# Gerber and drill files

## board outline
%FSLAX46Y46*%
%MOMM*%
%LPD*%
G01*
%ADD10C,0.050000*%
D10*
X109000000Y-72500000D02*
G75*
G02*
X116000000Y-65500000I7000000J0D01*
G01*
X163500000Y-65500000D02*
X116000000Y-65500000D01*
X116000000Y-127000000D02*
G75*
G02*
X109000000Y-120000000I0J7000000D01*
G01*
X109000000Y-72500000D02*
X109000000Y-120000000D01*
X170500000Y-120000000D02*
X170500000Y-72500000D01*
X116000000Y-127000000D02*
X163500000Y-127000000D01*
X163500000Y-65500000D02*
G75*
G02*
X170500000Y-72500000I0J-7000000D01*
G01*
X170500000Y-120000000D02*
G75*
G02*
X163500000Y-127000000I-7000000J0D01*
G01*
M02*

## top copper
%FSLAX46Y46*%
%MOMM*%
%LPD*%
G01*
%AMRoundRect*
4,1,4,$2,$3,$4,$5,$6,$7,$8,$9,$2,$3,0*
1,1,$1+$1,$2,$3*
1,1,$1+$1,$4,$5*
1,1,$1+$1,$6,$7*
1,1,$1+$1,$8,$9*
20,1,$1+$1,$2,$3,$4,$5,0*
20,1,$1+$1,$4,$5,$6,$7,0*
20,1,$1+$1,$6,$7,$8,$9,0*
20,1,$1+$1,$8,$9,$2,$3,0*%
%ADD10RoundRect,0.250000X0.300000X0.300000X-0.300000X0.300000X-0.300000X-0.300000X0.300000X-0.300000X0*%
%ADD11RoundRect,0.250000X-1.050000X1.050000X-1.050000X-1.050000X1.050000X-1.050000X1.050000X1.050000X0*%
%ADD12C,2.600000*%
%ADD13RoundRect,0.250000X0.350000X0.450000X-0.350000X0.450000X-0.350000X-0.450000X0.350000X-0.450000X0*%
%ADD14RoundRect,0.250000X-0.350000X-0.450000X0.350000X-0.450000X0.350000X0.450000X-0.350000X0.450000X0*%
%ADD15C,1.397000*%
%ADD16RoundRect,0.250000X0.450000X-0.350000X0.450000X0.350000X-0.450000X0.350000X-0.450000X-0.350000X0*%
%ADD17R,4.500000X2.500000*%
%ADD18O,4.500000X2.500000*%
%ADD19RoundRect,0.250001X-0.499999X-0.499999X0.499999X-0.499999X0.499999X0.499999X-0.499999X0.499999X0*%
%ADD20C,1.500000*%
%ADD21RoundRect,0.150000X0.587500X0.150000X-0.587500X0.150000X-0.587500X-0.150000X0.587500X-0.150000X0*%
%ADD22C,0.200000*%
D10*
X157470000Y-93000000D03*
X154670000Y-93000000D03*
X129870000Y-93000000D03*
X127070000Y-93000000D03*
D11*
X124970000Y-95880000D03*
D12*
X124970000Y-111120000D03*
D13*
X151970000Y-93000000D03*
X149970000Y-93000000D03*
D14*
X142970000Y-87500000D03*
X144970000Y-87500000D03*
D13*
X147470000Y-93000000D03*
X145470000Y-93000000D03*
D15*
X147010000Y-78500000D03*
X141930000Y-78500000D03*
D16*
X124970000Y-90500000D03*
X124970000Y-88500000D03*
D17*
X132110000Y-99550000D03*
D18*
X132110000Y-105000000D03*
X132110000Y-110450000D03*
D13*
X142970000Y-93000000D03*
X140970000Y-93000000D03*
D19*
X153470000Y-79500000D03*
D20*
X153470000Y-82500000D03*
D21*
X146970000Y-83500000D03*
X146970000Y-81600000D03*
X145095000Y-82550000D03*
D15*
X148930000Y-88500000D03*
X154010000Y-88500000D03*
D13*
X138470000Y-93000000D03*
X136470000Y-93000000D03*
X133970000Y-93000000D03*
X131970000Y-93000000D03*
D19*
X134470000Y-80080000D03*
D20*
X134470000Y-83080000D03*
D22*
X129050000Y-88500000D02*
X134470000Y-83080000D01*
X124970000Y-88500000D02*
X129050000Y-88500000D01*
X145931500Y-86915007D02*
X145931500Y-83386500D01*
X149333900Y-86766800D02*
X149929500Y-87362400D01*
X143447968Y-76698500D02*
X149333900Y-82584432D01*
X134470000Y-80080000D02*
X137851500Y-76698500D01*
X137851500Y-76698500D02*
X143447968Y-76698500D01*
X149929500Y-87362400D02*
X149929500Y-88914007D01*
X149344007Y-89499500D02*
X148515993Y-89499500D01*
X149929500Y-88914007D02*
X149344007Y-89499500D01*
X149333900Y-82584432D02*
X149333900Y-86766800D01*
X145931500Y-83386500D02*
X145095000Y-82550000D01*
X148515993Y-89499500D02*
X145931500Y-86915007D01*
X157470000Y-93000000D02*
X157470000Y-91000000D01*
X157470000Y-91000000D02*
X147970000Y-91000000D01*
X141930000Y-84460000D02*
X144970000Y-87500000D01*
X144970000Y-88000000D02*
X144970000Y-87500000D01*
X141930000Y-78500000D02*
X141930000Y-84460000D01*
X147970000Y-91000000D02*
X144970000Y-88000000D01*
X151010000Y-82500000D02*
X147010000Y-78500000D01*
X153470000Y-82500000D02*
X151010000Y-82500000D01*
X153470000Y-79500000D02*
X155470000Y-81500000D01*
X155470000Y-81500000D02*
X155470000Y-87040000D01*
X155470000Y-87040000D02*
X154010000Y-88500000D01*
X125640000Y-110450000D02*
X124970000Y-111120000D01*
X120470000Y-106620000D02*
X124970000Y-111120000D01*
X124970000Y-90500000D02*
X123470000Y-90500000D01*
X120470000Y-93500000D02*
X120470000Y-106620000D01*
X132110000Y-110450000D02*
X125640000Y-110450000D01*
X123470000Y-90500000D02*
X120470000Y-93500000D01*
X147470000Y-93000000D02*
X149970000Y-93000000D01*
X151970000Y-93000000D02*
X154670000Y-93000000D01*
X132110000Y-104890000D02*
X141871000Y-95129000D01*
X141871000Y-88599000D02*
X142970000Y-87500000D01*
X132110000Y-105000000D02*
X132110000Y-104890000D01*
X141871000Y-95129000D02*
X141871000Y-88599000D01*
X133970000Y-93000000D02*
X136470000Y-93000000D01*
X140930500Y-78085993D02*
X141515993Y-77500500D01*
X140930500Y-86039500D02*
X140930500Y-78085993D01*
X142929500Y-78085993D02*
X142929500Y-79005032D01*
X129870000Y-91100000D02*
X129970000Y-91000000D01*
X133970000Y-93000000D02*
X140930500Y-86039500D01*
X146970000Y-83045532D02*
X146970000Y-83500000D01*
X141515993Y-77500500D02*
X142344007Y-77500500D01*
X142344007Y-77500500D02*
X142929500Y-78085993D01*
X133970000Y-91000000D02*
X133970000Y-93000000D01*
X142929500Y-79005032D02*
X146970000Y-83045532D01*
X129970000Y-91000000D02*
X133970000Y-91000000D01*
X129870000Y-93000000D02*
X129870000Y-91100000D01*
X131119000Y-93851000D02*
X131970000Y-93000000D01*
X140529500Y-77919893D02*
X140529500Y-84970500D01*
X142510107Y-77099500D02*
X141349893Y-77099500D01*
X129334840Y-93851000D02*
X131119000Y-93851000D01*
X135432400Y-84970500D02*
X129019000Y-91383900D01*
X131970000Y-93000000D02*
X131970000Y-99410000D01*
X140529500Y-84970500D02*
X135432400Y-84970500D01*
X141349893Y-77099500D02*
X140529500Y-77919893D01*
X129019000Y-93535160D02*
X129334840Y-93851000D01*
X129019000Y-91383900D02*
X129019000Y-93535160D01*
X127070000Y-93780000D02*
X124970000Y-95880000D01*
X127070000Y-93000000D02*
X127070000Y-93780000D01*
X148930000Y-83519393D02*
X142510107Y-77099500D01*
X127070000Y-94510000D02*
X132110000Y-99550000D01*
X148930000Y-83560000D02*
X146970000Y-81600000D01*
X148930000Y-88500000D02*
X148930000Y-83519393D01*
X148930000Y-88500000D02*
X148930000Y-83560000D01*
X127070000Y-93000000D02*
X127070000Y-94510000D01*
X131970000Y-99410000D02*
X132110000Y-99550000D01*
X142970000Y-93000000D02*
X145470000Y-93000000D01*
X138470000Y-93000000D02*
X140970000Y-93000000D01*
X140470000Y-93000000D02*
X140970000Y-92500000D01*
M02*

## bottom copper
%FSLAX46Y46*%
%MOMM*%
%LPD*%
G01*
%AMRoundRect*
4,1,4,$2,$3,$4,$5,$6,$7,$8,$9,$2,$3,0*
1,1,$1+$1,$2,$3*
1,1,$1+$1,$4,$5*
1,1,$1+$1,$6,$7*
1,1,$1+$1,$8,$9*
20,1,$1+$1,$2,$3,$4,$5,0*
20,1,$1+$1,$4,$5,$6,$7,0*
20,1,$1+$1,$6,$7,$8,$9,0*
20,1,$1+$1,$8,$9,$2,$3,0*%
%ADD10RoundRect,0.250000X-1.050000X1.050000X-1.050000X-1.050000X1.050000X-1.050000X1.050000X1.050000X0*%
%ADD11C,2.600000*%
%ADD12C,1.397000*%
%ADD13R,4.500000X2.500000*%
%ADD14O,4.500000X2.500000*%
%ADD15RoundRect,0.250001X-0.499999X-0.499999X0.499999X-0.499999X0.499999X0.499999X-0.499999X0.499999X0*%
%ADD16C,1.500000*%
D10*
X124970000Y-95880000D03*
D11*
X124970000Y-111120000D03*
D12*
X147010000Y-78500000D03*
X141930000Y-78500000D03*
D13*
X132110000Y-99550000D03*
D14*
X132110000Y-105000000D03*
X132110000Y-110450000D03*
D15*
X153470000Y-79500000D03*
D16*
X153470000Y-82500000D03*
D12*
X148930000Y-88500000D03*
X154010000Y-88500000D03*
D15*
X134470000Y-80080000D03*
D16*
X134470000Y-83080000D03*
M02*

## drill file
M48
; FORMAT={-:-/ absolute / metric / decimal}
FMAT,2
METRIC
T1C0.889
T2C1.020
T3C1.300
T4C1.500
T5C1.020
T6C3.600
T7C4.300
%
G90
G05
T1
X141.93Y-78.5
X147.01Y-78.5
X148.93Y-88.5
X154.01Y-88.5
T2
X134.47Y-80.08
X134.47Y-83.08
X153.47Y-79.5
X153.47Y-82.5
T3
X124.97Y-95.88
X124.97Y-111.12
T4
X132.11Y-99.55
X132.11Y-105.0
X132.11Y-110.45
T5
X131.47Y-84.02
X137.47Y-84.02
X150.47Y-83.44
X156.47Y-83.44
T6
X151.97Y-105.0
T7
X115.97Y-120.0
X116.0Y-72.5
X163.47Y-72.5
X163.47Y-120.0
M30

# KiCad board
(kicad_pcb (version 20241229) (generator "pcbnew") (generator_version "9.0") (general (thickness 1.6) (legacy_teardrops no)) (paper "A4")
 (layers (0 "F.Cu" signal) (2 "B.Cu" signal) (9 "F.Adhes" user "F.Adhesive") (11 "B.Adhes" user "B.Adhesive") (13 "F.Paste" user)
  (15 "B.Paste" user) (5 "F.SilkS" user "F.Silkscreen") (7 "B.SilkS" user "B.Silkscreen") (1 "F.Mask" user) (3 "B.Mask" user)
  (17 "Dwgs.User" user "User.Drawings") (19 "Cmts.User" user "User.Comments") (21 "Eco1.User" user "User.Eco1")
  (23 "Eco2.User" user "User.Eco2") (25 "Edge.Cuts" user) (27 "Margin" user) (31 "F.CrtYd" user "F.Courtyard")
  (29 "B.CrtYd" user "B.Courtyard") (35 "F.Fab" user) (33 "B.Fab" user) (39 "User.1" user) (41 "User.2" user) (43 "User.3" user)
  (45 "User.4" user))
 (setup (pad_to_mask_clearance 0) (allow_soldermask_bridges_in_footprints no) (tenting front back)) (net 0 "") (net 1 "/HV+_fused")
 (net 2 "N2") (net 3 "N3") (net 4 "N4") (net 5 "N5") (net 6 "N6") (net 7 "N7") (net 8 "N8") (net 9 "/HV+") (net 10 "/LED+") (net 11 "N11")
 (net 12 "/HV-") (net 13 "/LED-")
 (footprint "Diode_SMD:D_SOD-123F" (layer "F.Cu") (at 156.07 93 180)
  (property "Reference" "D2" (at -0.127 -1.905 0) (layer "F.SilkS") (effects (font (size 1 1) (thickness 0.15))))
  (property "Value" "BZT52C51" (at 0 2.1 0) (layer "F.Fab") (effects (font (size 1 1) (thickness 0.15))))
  (pad "1" smd roundrect (at -1.4 0 180) (size 1.1 1.1) (layers "F.Cu" "F.Mask" "F.Paste") (roundrect_rratio 0.2272727273)
   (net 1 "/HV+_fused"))
  (pad "2" smd roundrect (at 1.4 0 180) (size 1.1 1.1) (layers "F.Cu" "F.Mask" "F.Paste") (roundrect_rratio 0.2272727273) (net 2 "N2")))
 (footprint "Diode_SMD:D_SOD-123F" (layer "F.Cu") (at 128.47 93 180)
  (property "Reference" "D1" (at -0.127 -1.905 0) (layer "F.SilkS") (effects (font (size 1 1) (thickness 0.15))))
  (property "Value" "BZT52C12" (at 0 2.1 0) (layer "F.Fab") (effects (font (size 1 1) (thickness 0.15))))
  (pad "1" smd roundrect (at -1.4 0 180) (size 1.1 1.1) (layers "F.Cu" "F.Mask" "F.Paste") (roundrect_rratio 0.2272727273) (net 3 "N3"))
  (pad "2" smd roundrect (at 1.4 0 180) (size 1.1 1.1) (layers "F.Cu" "F.Mask" "F.Paste") (roundrect_rratio 0.2272727273) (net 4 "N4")))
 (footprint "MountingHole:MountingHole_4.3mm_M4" (layer "F.Cu") (at 116 72.5)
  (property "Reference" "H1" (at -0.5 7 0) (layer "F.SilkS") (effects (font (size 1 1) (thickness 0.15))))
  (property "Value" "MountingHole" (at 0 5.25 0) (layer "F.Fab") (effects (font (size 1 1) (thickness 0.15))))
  (pad "" np_thru_hole circle (at 0 0) (size 4.3 4.3) (drill 4.3) (layers "*.Cu" "*.Mask")))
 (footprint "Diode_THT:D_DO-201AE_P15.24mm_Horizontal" (layer "F.Cu") (at 124.97 95.88 -90)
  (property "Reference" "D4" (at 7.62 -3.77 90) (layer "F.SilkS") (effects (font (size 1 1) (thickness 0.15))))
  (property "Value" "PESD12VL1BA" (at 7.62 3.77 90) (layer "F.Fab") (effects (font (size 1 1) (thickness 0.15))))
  (pad "1" thru_hole roundrect (at 0 0 270) (size 2.6 2.6) (drill 1.3) (layers "*.Cu" "*.Mask") (remove_unused_layers no)
   (roundrect_rratio 0.096154) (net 4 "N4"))
  (pad "2" thru_hole circle (at 15.24 0 270) (size 2.6 2.6) (drill 1.3) (layers "*.Cu" "*.Mask") (remove_unused_layers no) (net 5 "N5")))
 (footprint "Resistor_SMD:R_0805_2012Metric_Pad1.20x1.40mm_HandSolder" (layer "F.Cu") (at 150.97 93 180)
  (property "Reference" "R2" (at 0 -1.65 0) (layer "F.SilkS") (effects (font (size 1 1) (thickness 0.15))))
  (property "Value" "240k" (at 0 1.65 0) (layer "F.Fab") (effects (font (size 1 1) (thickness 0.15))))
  (pad "1" smd roundrect (at -1 0 180) (size 1.2 1.4) (layers "F.Cu" "F.Mask" "F.Paste") (roundrect_rratio 0.208333) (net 2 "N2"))
  (pad "2" smd roundrect (at 1 0 180) (size 1.2 1.4) (layers "F.Cu" "F.Mask" "F.Paste") (roundrect_rratio 0.208333) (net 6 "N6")))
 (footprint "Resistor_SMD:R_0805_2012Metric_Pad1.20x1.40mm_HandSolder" (layer "F.Cu") (at 143.97 87.5)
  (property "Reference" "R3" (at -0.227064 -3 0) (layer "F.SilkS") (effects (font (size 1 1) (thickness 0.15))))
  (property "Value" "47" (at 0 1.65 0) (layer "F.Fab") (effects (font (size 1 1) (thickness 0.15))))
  (pad "1" smd roundrect (at -1 0) (size 1.2 1.4) (layers "F.Cu" "F.Mask" "F.Paste") (roundrect_rratio 0.208333) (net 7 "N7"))
  (pad "2" smd roundrect (at 1 0) (size 1.2 1.4) (layers "F.Cu" "F.Mask" "F.Paste") (roundrect_rratio 0.208333) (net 1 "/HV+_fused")))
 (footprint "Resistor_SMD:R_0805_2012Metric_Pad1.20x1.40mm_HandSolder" (layer "F.Cu") (at 146.47 93 180)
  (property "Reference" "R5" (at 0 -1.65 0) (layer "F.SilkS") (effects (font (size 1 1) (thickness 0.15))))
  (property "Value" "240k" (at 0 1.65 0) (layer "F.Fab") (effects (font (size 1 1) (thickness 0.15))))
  (pad "1" smd roundrect (at -1 0 180) (size 1.2 1.4) (layers "F.Cu" "F.Mask" "F.Paste") (roundrect_rratio 0.208333) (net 6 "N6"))
  (pad "2" smd roundrect (at 1 0 180) (size 1.2 1.4) (layers "F.Cu" "F.Mask" "F.Paste") (roundrect_rratio 0.208333) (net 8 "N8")))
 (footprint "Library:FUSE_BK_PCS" (layer "F.Cu") (at 144.47 78.5 180)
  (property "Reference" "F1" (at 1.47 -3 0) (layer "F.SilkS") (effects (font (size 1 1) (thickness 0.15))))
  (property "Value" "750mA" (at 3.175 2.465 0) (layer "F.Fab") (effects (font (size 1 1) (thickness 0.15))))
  (pad "1" thru_hole circle (at -2.54 0 180) (size 1.397 1.397) (drill 0.889) (layers "*.Cu" "*.Mask") (remove_unused_layers no)
   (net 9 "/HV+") (solder_mask_margin 0.102))
  (pad "2" thru_hole circle (at 2.54 0 180) (size 1.397 1.397) (drill 0.889) (layers "*.Cu" "*.Mask") (remove_unused_layers no)
   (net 1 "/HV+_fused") (solder_mask_margin 0.102)))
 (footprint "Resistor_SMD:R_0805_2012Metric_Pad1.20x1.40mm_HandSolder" (layer "F.Cu") (at 124.97 89.5 90)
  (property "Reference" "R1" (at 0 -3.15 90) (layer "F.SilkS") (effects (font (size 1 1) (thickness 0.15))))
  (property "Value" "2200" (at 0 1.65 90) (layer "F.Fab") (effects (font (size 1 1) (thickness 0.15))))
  (pad "1" smd roundrect (at -1 0 90) (size 1.2 1.4) (layers "F.Cu" "F.Mask" "F.Paste") (roundrect_rratio 0.208333) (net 5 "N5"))
  (pad "2" smd roundrect (at 1 0 90) (size 1.2 1.4) (layers "F.Cu" "F.Mask" "F.Paste") (roundrect_rratio 0.208333) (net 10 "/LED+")))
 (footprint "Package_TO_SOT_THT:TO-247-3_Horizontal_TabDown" (layer "F.Cu") (at 132.11 99.55 -90)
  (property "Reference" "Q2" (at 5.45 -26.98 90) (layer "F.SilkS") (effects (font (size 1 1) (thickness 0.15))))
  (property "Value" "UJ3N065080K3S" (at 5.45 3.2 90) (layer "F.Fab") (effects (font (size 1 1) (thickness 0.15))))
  (pad "" np_thru_hole circle (at 5.45 -19.86 270) (size 3.6 3.6) (drill 3.6) (layers "*.Cu" "*.Mask"))
  (pad "1" thru_hole rect (at 0 0 270) (size 2.5 4.5) (drill 1.5) (layers "*.Cu" "*.Mask") (remove_unused_layers no) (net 4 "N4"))
  (pad "2" thru_hole oval (at 5.45 0 270) (size 2.5 4.5) (drill 1.5) (layers "*.Cu" "*.Mask") (remove_unused_layers no) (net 7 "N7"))
  (pad "3" thru_hole oval (at 10.9 0 270) (size 2.5 4.5) (drill 1.5) (layers "*.Cu" "*.Mask") (remove_unused_layers no) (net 5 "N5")))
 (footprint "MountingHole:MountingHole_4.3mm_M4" (layer "F.Cu") (at 115.97 120)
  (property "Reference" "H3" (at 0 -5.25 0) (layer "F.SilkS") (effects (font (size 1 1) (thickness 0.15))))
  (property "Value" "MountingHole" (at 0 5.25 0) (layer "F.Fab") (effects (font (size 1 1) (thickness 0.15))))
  (pad "" np_thru_hole circle (at 0 0) (size 4.3 4.3) (drill 4.3) (layers "*.Cu" "*.Mask")))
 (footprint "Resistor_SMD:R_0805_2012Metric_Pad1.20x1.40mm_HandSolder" (layer "F.Cu") (at 141.97 93 180)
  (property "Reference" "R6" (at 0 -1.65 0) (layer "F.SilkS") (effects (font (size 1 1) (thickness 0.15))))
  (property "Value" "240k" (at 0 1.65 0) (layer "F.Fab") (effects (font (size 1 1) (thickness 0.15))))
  (pad "1" smd roundrect (at -1 0 180) (size 1.2 1.4) (layers "F.Cu" "F.Mask" "F.Paste") (roundrect_rratio 0.208333) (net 8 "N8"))
  (pad "2" smd roundrect (at 1 0 180) (size 1.2 1.4) (layers "F.Cu" "F.Mask" "F.Paste") (roundrect_rratio 0.208333) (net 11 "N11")))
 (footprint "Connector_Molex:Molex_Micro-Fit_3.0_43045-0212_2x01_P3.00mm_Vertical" (layer "F.Cu") (at 153.47 79.5)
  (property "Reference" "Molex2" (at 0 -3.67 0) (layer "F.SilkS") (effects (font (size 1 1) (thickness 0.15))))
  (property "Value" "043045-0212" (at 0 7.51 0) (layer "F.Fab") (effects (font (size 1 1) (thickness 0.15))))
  (pad "" np_thru_hole circle (at -3 3.94) (size 1.02 1.02) (drill 1.02) (layers "*.Cu" "*.Mask"))
  (pad "" np_thru_hole circle (at 3 3.94) (size 1.02 1.02) (drill 1.02) (layers "*.Cu" "*.Mask"))
  (pad "1" thru_hole roundrect (at 0 0) (size 1.5 1.5) (drill 1.02) (layers "*.Cu" "*.Mask") (remove_unused_layers no)
   (roundrect_rratio 0.166667) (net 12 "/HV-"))
  (pad "2" thru_hole circle (at 0 3) (size 1.5 1.5) (drill 1.02) (layers "*.Cu" "*.Mask") (remove_unused_layers no) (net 9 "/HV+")))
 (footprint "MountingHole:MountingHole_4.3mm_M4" (layer "F.Cu") (at 163.47 72.5)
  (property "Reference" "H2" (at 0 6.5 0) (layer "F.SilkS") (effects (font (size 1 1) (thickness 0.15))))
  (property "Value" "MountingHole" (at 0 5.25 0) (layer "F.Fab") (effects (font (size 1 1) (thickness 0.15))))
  (pad "" np_thru_hole circle (at 0 0) (size 4.3 4.3) (drill 4.3) (layers "*.Cu" "*.Mask")))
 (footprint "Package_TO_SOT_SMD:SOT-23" (layer "F.Cu") (at 146.0325 82.55 180)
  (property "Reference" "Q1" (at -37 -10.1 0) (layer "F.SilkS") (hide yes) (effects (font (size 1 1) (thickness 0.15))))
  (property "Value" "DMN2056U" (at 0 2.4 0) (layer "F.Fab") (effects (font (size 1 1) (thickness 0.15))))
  (pad "1" smd roundrect (at -0.9375 -0.95 180) (size 1.475 0.6) (layers "F.Cu" "F.Mask" "F.Paste") (roundrect_rratio 0.25) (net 3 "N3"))
  (pad "2" smd roundrect (at -0.9375 0.95 180) (size 1.475 0.6) (layers "F.Cu" "F.Mask" "F.Paste") (roundrect_rratio 0.25) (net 4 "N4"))
  (pad "3" smd roundrect (at 0.9375 0 180) (size 1.475 0.6) (layers "F.Cu" "F.Mask" "F.Paste") (roundrect_rratio 0.25) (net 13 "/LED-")))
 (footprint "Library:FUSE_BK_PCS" (layer "F.Cu") (at 151.47 88.5)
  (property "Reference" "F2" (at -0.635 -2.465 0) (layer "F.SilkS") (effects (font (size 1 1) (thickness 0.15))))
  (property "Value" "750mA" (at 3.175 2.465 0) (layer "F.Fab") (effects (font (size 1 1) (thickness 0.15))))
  (pad "1" thru_hole circle (at -2.54 0) (size 1.397 1.397) (drill 0.889) (layers "*.Cu" "*.Mask") (remove_unused_layers no) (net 4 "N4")
   (solder_mask_margin 0.102))
  (pad "2" thru_hole circle (at 2.54 0) (size 1.397 1.397) (drill 0.889) (layers "*.Cu" "*.Mask") (remove_unused_layers no) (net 12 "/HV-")
   (solder_mask_margin 0.102)))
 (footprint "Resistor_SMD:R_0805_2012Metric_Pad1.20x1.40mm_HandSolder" (layer "F.Cu") (at 137.47 93 180)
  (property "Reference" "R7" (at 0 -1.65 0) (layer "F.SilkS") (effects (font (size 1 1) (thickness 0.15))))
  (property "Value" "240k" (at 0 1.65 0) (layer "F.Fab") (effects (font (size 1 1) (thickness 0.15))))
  (pad "1" smd roundrect (at -1 0 180) (size 1.2 1.4) (layers "F.Cu" "F.Mask" "F.Paste") (roundrect_rratio 0.208333) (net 11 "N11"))
  (pad "2" smd roundrect (at 1 0 180) (size 1.2 1.4) (layers "F.Cu" "F.Mask" "F.Paste") (roundrect_rratio 0.208333) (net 3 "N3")))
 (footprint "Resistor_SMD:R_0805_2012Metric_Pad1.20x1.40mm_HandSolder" (layer "F.Cu") (at 132.97 93 180)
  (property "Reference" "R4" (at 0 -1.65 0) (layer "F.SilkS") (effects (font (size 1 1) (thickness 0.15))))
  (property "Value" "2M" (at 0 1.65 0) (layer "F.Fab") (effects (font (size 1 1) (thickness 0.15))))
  (pad "1" smd roundrect (at -1 0 180) (size 1.2 1.4) (layers "F.Cu" "F.Mask" "F.Paste") (roundrect_rratio 0.208333) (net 3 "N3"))
  (pad "2" smd roundrect (at 1 0 180) (size 1.2 1.4) (layers "F.Cu" "F.Mask" "F.Paste") (roundrect_rratio 0.208333) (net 4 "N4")))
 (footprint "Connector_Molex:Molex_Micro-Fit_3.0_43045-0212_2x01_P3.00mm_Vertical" (layer "F.Cu") (at 134.47 80.08)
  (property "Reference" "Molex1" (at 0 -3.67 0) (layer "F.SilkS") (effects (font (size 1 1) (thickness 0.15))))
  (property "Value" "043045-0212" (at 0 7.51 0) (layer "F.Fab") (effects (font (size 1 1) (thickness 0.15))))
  (pad "" np_thru_hole circle (at -3 3.94) (size 1.02 1.02) (drill 1.02) (layers "*.Cu" "*.Mask"))
  (pad "" np_thru_hole circle (at 3 3.94) (size 1.02 1.02) (drill 1.02) (layers "*.Cu" "*.Mask"))
  (pad "1" thru_hole roundrect (at 0 0) (size 1.5 1.5) (drill 1.02) (layers "*.Cu" "*.Mask") (remove_unused_layers no)
   (roundrect_rratio 0.166667) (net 13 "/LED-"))
  (pad "2" thru_hole circle (at 0 3) (size 1.5 1.5) (drill 1.02) (layers "*.Cu" "*.Mask") (remove_unused_layers no) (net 10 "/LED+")))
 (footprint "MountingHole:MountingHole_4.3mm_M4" (layer "F.Cu") (at 163.47 120)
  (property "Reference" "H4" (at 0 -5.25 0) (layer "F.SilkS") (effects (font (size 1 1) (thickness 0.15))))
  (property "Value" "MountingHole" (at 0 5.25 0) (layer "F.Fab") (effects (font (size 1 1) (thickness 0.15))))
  (pad "" np_thru_hole circle (at 0 0) (size 4.3 4.3) (drill 4.3) (layers "*.Cu" "*.Mask")))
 (gr_arc (start 109 72.5) (mid 111.050253 67.550253) (end 116 65.5) (stroke (width 0.05) (type default)) (layer "Edge.Cuts"))
 (gr_line (start 163.5 65.5) (end 116 65.5) (stroke (width 0.05) (type default)) (layer "Edge.Cuts"))
 (gr_arc (start 116 127) (mid 111.050253 124.949747) (end 109 120) (stroke (width 0.05) (type default)) (layer "Edge.Cuts"))
 (gr_line (start 109 72.5) (end 109 120) (stroke (width 0.05) (type default)) (layer "Edge.Cuts"))
 (gr_line (start 170.5 120) (end 170.5 72.5) (stroke (width 0.05) (type default)) (layer "Edge.Cuts"))
 (gr_line (start 116 127) (end 163.5 127) (stroke (width 0.05) (type default)) (layer "Edge.Cuts"))
 (gr_arc (start 163.5 65.5) (mid 168.449747 67.550253) (end 170.5 72.5) (stroke (width 0.05) (type default)) (layer "Edge.Cuts"))
 (gr_arc (start 170.5 120) (mid 168.449747 124.949747) (end 163.5 127) (stroke (width 0.05) (type default)) (layer "Edge.Cuts"))
 (segment (start 129.05 88.5) (end 134.47 83.08) (width 0.2) (layer "F.Cu") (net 10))
 (segment (start 124.97 88.5) (end 129.05 88.5) (width 0.2) (layer "F.Cu") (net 10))
 (segment (start 145.9315 86.915007) (end 145.9315 83.3865) (width 0.2) (layer "F.Cu") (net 13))
 (segment (start 149.3339 86.7668) (end 149.9295 87.3624) (width 0.2) (layer "F.Cu") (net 13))
 (segment (start 143.447968 76.6985) (end 149.3339 82.584432) (width 0.2) (layer "F.Cu") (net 13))
 (segment (start 134.47 80.08) (end 137.8515 76.6985) (width 0.2) (layer "F.Cu") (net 13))
 (segment (start 137.8515 76.6985) (end 143.447968 76.6985) (width 0.2) (layer "F.Cu") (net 13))
 (segment (start 149.9295 87.3624) (end 149.9295 88.914007) (width 0.2) (layer "F.Cu") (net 13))
 (segment (start 149.344007 89.4995) (end 148.515993 89.4995) (width 0.2) (layer "F.Cu") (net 13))
 (segment (start 149.9295 88.914007) (end 149.344007 89.4995) (width 0.2) (layer "F.Cu") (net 13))
 (segment (start 149.3339 82.584432) (end 149.3339 86.7668) (width 0.2) (layer "F.Cu") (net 13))
 (segment (start 145.9315 83.3865) (end 145.095 82.55) (width 0.2) (layer "F.Cu") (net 13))
 (segment (start 148.515993 89.4995) (end 145.9315 86.915007) (width 0.2) (layer "F.Cu") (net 13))
 (segment (start 157.47 93) (end 157.47 91) (width 0.2) (layer "F.Cu") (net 1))
 (segment (start 157.47 91) (end 147.97 91) (width 0.2) (layer "F.Cu") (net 1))
 (segment (start 141.93 84.46) (end 144.97 87.5) (width 0.2) (layer "F.Cu") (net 1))
 (segment (start 144.97 88) (end 144.97 87.5) (width 0.2) (layer "F.Cu") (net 1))
 (segment (start 141.93 78.5) (end 141.93 84.46) (width 0.2) (layer "F.Cu") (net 1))
 (segment (start 147.97 91) (end 144.97 88) (width 0.2) (layer "F.Cu") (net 1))
 (segment (start 151.01 82.5) (end 147.01 78.5) (width 0.2) (layer "F.Cu") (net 9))
 (segment (start 153.47 82.5) (end 151.01 82.5) (width 0.2) (layer "F.Cu") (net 9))
 (segment (start 153.47 79.5) (end 155.47 81.5) (width 0.2) (layer "F.Cu") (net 12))
 (segment (start 155.47 81.5) (end 155.47 87.04) (width 0.2) (layer "F.Cu") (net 12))
 (segment (start 155.47 87.04) (end 154.01 88.5) (width 0.2) (layer "F.Cu") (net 12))
 (segment (start 125.64 110.45) (end 124.97 111.12) (width 0.2) (layer "F.Cu") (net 5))
 (segment (start 120.47 106.62) (end 124.97 111.12) (width 0.2) (layer "F.Cu") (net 5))
 (segment (start 124.97 90.5) (end 123.47 90.5) (width 0.2) (layer "F.Cu") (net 5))
 (segment (start 120.47 93.5) (end 120.47 106.62) (width 0.2) (layer "F.Cu") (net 5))
 (segment (start 132.11 110.45) (end 125.64 110.45) (width 0.2) (layer "F.Cu") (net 5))
 (segment (start 123.47 90.5) (end 120.47 93.5) (width 0.2) (layer "F.Cu") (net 5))
 (segment (start 147.47 93) (end 149.97 93) (width 0.2) (layer "F.Cu") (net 6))
 (segment (start 151.97 93) (end 154.67 93) (width 0.2) (layer "F.Cu") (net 2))
 (segment (start 132.11 104.89) (end 141.871 95.129) (width 0.2) (layer "F.Cu") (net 7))
 (segment (start 141.871 88.599) (end 142.97 87.5) (width 0.2) (layer "F.Cu") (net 7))
 (segment (start 132.11 105) (end 132.11 104.89) (width 0.2) (layer "F.Cu") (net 7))
 (segment (start 141.871 95.129) (end 141.871 88.599) (width 0.2) (layer "F.Cu") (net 7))
 (segment (start 133.97 93) (end 136.47 93) (width 0.2) (layer "F.Cu") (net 3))
 (segment (start 140.9305 78.085993) (end 141.515993 77.5005) (width 0.2) (layer "F.Cu") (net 3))
 (segment (start 140.9305 86.0395) (end 140.9305 78.085993) (width 0.2) (layer "F.Cu") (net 3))
 (segment (start 142.9295 78.085993) (end 142.9295 79.005032) (width 0.2) (layer "F.Cu") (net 3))
 (segment (start 129.87 91.1) (end 129.97 91) (width 0.2) (layer "F.Cu") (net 3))
 (segment (start 133.97 93) (end 140.9305 86.0395) (width 0.2) (layer "F.Cu") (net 3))
 (segment (start 146.97 83.045532) (end 146.97 83.5) (width 0.2) (layer "F.Cu") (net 3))
 (segment (start 141.515993 77.5005) (end 142.344007 77.5005) (width 0.2) (layer "F.Cu") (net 3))
 (segment (start 142.344007 77.5005) (end 142.9295 78.085993) (width 0.2) (layer "F.Cu") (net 3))
 (segment (start 133.97 91) (end 133.97 93) (width 0.2) (layer "F.Cu") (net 3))
 (segment (start 142.9295 79.005032) (end 146.97 83.045532) (width 0.2) (layer "F.Cu") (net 3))
 (segment (start 129.97 91) (end 133.97 91) (width 0.2) (layer "F.Cu") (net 3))
 (segment (start 129.87 93) (end 129.87 91.1) (width 0.2) (layer "F.Cu") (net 3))
 (segment (start 131.119 93.851) (end 131.97 93) (width 0.2) (layer "F.Cu") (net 4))
 (segment (start 140.5295 77.919893) (end 140.5295 84.9705) (width 0.2) (layer "F.Cu") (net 4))
 (segment (start 142.510107 77.0995) (end 141.349893 77.0995) (width 0.2) (layer "F.Cu") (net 4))
 (segment (start 129.33484 93.851) (end 131.119 93.851) (width 0.2) (layer "F.Cu") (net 4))
 (segment (start 135.4324 84.9705) (end 129.019 91.3839) (width 0.2) (layer "F.Cu") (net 4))
 (segment (start 131.97 93) (end 131.97 99.41) (width 0.2) (layer "F.Cu") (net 4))
 (segment (start 140.5295 84.9705) (end 135.4324 84.9705) (width 0.2) (layer "F.Cu") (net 4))
 (segment (start 141.349893 77.0995) (end 140.5295 77.919893) (width 0.2) (layer "F.Cu") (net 4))
 (segment (start 129.019 93.53516) (end 129.33484 93.851) (width 0.2) (layer "F.Cu") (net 4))
 (segment (start 129.019 91.3839) (end 129.019 93.53516) (width 0.2) (layer "F.Cu") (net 4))
 (segment (start 127.07 93.78) (end 124.97 95.88) (width 0.2) (layer "F.Cu") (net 4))
 (segment (start 127.07 93) (end 127.07 93.78) (width 0.2) (layer "F.Cu") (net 4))
 (segment (start 148.93 83.519393) (end 142.510107 77.0995) (width 0.2) (layer "F.Cu") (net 4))
 (segment (start 127.07 94.51) (end 132.11 99.55) (width 0.2) (layer "F.Cu") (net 4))
 (segment (start 148.93 83.56) (end 146.97 81.6) (width 0.2) (layer "F.Cu") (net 4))
 (segment (start 148.93 88.5) (end 148.93 83.519393) (width 0.2) (layer "F.Cu") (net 4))
 (segment (start 148.93 88.5) (end 148.93 83.56) (width 0.2) (layer "F.Cu") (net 4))
 (segment (start 127.07 93) (end 127.07 94.51) (width 0.2) (layer "F.Cu") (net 4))
 (segment (start 131.97 99.41) (end 132.11 99.55) (width 0.2) (layer "F.Cu") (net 4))
 (segment (start 142.97 93) (end 145.47 93) (width 0.2) (layer "F.Cu") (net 8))
 (segment (start 138.47 93) (end 140.97 93) (width 0.2) (layer "F.Cu") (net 11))
 (segment (start 140.47 93) (end 140.97 92.5) (width 0.2) (layer "F.Cu") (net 11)))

